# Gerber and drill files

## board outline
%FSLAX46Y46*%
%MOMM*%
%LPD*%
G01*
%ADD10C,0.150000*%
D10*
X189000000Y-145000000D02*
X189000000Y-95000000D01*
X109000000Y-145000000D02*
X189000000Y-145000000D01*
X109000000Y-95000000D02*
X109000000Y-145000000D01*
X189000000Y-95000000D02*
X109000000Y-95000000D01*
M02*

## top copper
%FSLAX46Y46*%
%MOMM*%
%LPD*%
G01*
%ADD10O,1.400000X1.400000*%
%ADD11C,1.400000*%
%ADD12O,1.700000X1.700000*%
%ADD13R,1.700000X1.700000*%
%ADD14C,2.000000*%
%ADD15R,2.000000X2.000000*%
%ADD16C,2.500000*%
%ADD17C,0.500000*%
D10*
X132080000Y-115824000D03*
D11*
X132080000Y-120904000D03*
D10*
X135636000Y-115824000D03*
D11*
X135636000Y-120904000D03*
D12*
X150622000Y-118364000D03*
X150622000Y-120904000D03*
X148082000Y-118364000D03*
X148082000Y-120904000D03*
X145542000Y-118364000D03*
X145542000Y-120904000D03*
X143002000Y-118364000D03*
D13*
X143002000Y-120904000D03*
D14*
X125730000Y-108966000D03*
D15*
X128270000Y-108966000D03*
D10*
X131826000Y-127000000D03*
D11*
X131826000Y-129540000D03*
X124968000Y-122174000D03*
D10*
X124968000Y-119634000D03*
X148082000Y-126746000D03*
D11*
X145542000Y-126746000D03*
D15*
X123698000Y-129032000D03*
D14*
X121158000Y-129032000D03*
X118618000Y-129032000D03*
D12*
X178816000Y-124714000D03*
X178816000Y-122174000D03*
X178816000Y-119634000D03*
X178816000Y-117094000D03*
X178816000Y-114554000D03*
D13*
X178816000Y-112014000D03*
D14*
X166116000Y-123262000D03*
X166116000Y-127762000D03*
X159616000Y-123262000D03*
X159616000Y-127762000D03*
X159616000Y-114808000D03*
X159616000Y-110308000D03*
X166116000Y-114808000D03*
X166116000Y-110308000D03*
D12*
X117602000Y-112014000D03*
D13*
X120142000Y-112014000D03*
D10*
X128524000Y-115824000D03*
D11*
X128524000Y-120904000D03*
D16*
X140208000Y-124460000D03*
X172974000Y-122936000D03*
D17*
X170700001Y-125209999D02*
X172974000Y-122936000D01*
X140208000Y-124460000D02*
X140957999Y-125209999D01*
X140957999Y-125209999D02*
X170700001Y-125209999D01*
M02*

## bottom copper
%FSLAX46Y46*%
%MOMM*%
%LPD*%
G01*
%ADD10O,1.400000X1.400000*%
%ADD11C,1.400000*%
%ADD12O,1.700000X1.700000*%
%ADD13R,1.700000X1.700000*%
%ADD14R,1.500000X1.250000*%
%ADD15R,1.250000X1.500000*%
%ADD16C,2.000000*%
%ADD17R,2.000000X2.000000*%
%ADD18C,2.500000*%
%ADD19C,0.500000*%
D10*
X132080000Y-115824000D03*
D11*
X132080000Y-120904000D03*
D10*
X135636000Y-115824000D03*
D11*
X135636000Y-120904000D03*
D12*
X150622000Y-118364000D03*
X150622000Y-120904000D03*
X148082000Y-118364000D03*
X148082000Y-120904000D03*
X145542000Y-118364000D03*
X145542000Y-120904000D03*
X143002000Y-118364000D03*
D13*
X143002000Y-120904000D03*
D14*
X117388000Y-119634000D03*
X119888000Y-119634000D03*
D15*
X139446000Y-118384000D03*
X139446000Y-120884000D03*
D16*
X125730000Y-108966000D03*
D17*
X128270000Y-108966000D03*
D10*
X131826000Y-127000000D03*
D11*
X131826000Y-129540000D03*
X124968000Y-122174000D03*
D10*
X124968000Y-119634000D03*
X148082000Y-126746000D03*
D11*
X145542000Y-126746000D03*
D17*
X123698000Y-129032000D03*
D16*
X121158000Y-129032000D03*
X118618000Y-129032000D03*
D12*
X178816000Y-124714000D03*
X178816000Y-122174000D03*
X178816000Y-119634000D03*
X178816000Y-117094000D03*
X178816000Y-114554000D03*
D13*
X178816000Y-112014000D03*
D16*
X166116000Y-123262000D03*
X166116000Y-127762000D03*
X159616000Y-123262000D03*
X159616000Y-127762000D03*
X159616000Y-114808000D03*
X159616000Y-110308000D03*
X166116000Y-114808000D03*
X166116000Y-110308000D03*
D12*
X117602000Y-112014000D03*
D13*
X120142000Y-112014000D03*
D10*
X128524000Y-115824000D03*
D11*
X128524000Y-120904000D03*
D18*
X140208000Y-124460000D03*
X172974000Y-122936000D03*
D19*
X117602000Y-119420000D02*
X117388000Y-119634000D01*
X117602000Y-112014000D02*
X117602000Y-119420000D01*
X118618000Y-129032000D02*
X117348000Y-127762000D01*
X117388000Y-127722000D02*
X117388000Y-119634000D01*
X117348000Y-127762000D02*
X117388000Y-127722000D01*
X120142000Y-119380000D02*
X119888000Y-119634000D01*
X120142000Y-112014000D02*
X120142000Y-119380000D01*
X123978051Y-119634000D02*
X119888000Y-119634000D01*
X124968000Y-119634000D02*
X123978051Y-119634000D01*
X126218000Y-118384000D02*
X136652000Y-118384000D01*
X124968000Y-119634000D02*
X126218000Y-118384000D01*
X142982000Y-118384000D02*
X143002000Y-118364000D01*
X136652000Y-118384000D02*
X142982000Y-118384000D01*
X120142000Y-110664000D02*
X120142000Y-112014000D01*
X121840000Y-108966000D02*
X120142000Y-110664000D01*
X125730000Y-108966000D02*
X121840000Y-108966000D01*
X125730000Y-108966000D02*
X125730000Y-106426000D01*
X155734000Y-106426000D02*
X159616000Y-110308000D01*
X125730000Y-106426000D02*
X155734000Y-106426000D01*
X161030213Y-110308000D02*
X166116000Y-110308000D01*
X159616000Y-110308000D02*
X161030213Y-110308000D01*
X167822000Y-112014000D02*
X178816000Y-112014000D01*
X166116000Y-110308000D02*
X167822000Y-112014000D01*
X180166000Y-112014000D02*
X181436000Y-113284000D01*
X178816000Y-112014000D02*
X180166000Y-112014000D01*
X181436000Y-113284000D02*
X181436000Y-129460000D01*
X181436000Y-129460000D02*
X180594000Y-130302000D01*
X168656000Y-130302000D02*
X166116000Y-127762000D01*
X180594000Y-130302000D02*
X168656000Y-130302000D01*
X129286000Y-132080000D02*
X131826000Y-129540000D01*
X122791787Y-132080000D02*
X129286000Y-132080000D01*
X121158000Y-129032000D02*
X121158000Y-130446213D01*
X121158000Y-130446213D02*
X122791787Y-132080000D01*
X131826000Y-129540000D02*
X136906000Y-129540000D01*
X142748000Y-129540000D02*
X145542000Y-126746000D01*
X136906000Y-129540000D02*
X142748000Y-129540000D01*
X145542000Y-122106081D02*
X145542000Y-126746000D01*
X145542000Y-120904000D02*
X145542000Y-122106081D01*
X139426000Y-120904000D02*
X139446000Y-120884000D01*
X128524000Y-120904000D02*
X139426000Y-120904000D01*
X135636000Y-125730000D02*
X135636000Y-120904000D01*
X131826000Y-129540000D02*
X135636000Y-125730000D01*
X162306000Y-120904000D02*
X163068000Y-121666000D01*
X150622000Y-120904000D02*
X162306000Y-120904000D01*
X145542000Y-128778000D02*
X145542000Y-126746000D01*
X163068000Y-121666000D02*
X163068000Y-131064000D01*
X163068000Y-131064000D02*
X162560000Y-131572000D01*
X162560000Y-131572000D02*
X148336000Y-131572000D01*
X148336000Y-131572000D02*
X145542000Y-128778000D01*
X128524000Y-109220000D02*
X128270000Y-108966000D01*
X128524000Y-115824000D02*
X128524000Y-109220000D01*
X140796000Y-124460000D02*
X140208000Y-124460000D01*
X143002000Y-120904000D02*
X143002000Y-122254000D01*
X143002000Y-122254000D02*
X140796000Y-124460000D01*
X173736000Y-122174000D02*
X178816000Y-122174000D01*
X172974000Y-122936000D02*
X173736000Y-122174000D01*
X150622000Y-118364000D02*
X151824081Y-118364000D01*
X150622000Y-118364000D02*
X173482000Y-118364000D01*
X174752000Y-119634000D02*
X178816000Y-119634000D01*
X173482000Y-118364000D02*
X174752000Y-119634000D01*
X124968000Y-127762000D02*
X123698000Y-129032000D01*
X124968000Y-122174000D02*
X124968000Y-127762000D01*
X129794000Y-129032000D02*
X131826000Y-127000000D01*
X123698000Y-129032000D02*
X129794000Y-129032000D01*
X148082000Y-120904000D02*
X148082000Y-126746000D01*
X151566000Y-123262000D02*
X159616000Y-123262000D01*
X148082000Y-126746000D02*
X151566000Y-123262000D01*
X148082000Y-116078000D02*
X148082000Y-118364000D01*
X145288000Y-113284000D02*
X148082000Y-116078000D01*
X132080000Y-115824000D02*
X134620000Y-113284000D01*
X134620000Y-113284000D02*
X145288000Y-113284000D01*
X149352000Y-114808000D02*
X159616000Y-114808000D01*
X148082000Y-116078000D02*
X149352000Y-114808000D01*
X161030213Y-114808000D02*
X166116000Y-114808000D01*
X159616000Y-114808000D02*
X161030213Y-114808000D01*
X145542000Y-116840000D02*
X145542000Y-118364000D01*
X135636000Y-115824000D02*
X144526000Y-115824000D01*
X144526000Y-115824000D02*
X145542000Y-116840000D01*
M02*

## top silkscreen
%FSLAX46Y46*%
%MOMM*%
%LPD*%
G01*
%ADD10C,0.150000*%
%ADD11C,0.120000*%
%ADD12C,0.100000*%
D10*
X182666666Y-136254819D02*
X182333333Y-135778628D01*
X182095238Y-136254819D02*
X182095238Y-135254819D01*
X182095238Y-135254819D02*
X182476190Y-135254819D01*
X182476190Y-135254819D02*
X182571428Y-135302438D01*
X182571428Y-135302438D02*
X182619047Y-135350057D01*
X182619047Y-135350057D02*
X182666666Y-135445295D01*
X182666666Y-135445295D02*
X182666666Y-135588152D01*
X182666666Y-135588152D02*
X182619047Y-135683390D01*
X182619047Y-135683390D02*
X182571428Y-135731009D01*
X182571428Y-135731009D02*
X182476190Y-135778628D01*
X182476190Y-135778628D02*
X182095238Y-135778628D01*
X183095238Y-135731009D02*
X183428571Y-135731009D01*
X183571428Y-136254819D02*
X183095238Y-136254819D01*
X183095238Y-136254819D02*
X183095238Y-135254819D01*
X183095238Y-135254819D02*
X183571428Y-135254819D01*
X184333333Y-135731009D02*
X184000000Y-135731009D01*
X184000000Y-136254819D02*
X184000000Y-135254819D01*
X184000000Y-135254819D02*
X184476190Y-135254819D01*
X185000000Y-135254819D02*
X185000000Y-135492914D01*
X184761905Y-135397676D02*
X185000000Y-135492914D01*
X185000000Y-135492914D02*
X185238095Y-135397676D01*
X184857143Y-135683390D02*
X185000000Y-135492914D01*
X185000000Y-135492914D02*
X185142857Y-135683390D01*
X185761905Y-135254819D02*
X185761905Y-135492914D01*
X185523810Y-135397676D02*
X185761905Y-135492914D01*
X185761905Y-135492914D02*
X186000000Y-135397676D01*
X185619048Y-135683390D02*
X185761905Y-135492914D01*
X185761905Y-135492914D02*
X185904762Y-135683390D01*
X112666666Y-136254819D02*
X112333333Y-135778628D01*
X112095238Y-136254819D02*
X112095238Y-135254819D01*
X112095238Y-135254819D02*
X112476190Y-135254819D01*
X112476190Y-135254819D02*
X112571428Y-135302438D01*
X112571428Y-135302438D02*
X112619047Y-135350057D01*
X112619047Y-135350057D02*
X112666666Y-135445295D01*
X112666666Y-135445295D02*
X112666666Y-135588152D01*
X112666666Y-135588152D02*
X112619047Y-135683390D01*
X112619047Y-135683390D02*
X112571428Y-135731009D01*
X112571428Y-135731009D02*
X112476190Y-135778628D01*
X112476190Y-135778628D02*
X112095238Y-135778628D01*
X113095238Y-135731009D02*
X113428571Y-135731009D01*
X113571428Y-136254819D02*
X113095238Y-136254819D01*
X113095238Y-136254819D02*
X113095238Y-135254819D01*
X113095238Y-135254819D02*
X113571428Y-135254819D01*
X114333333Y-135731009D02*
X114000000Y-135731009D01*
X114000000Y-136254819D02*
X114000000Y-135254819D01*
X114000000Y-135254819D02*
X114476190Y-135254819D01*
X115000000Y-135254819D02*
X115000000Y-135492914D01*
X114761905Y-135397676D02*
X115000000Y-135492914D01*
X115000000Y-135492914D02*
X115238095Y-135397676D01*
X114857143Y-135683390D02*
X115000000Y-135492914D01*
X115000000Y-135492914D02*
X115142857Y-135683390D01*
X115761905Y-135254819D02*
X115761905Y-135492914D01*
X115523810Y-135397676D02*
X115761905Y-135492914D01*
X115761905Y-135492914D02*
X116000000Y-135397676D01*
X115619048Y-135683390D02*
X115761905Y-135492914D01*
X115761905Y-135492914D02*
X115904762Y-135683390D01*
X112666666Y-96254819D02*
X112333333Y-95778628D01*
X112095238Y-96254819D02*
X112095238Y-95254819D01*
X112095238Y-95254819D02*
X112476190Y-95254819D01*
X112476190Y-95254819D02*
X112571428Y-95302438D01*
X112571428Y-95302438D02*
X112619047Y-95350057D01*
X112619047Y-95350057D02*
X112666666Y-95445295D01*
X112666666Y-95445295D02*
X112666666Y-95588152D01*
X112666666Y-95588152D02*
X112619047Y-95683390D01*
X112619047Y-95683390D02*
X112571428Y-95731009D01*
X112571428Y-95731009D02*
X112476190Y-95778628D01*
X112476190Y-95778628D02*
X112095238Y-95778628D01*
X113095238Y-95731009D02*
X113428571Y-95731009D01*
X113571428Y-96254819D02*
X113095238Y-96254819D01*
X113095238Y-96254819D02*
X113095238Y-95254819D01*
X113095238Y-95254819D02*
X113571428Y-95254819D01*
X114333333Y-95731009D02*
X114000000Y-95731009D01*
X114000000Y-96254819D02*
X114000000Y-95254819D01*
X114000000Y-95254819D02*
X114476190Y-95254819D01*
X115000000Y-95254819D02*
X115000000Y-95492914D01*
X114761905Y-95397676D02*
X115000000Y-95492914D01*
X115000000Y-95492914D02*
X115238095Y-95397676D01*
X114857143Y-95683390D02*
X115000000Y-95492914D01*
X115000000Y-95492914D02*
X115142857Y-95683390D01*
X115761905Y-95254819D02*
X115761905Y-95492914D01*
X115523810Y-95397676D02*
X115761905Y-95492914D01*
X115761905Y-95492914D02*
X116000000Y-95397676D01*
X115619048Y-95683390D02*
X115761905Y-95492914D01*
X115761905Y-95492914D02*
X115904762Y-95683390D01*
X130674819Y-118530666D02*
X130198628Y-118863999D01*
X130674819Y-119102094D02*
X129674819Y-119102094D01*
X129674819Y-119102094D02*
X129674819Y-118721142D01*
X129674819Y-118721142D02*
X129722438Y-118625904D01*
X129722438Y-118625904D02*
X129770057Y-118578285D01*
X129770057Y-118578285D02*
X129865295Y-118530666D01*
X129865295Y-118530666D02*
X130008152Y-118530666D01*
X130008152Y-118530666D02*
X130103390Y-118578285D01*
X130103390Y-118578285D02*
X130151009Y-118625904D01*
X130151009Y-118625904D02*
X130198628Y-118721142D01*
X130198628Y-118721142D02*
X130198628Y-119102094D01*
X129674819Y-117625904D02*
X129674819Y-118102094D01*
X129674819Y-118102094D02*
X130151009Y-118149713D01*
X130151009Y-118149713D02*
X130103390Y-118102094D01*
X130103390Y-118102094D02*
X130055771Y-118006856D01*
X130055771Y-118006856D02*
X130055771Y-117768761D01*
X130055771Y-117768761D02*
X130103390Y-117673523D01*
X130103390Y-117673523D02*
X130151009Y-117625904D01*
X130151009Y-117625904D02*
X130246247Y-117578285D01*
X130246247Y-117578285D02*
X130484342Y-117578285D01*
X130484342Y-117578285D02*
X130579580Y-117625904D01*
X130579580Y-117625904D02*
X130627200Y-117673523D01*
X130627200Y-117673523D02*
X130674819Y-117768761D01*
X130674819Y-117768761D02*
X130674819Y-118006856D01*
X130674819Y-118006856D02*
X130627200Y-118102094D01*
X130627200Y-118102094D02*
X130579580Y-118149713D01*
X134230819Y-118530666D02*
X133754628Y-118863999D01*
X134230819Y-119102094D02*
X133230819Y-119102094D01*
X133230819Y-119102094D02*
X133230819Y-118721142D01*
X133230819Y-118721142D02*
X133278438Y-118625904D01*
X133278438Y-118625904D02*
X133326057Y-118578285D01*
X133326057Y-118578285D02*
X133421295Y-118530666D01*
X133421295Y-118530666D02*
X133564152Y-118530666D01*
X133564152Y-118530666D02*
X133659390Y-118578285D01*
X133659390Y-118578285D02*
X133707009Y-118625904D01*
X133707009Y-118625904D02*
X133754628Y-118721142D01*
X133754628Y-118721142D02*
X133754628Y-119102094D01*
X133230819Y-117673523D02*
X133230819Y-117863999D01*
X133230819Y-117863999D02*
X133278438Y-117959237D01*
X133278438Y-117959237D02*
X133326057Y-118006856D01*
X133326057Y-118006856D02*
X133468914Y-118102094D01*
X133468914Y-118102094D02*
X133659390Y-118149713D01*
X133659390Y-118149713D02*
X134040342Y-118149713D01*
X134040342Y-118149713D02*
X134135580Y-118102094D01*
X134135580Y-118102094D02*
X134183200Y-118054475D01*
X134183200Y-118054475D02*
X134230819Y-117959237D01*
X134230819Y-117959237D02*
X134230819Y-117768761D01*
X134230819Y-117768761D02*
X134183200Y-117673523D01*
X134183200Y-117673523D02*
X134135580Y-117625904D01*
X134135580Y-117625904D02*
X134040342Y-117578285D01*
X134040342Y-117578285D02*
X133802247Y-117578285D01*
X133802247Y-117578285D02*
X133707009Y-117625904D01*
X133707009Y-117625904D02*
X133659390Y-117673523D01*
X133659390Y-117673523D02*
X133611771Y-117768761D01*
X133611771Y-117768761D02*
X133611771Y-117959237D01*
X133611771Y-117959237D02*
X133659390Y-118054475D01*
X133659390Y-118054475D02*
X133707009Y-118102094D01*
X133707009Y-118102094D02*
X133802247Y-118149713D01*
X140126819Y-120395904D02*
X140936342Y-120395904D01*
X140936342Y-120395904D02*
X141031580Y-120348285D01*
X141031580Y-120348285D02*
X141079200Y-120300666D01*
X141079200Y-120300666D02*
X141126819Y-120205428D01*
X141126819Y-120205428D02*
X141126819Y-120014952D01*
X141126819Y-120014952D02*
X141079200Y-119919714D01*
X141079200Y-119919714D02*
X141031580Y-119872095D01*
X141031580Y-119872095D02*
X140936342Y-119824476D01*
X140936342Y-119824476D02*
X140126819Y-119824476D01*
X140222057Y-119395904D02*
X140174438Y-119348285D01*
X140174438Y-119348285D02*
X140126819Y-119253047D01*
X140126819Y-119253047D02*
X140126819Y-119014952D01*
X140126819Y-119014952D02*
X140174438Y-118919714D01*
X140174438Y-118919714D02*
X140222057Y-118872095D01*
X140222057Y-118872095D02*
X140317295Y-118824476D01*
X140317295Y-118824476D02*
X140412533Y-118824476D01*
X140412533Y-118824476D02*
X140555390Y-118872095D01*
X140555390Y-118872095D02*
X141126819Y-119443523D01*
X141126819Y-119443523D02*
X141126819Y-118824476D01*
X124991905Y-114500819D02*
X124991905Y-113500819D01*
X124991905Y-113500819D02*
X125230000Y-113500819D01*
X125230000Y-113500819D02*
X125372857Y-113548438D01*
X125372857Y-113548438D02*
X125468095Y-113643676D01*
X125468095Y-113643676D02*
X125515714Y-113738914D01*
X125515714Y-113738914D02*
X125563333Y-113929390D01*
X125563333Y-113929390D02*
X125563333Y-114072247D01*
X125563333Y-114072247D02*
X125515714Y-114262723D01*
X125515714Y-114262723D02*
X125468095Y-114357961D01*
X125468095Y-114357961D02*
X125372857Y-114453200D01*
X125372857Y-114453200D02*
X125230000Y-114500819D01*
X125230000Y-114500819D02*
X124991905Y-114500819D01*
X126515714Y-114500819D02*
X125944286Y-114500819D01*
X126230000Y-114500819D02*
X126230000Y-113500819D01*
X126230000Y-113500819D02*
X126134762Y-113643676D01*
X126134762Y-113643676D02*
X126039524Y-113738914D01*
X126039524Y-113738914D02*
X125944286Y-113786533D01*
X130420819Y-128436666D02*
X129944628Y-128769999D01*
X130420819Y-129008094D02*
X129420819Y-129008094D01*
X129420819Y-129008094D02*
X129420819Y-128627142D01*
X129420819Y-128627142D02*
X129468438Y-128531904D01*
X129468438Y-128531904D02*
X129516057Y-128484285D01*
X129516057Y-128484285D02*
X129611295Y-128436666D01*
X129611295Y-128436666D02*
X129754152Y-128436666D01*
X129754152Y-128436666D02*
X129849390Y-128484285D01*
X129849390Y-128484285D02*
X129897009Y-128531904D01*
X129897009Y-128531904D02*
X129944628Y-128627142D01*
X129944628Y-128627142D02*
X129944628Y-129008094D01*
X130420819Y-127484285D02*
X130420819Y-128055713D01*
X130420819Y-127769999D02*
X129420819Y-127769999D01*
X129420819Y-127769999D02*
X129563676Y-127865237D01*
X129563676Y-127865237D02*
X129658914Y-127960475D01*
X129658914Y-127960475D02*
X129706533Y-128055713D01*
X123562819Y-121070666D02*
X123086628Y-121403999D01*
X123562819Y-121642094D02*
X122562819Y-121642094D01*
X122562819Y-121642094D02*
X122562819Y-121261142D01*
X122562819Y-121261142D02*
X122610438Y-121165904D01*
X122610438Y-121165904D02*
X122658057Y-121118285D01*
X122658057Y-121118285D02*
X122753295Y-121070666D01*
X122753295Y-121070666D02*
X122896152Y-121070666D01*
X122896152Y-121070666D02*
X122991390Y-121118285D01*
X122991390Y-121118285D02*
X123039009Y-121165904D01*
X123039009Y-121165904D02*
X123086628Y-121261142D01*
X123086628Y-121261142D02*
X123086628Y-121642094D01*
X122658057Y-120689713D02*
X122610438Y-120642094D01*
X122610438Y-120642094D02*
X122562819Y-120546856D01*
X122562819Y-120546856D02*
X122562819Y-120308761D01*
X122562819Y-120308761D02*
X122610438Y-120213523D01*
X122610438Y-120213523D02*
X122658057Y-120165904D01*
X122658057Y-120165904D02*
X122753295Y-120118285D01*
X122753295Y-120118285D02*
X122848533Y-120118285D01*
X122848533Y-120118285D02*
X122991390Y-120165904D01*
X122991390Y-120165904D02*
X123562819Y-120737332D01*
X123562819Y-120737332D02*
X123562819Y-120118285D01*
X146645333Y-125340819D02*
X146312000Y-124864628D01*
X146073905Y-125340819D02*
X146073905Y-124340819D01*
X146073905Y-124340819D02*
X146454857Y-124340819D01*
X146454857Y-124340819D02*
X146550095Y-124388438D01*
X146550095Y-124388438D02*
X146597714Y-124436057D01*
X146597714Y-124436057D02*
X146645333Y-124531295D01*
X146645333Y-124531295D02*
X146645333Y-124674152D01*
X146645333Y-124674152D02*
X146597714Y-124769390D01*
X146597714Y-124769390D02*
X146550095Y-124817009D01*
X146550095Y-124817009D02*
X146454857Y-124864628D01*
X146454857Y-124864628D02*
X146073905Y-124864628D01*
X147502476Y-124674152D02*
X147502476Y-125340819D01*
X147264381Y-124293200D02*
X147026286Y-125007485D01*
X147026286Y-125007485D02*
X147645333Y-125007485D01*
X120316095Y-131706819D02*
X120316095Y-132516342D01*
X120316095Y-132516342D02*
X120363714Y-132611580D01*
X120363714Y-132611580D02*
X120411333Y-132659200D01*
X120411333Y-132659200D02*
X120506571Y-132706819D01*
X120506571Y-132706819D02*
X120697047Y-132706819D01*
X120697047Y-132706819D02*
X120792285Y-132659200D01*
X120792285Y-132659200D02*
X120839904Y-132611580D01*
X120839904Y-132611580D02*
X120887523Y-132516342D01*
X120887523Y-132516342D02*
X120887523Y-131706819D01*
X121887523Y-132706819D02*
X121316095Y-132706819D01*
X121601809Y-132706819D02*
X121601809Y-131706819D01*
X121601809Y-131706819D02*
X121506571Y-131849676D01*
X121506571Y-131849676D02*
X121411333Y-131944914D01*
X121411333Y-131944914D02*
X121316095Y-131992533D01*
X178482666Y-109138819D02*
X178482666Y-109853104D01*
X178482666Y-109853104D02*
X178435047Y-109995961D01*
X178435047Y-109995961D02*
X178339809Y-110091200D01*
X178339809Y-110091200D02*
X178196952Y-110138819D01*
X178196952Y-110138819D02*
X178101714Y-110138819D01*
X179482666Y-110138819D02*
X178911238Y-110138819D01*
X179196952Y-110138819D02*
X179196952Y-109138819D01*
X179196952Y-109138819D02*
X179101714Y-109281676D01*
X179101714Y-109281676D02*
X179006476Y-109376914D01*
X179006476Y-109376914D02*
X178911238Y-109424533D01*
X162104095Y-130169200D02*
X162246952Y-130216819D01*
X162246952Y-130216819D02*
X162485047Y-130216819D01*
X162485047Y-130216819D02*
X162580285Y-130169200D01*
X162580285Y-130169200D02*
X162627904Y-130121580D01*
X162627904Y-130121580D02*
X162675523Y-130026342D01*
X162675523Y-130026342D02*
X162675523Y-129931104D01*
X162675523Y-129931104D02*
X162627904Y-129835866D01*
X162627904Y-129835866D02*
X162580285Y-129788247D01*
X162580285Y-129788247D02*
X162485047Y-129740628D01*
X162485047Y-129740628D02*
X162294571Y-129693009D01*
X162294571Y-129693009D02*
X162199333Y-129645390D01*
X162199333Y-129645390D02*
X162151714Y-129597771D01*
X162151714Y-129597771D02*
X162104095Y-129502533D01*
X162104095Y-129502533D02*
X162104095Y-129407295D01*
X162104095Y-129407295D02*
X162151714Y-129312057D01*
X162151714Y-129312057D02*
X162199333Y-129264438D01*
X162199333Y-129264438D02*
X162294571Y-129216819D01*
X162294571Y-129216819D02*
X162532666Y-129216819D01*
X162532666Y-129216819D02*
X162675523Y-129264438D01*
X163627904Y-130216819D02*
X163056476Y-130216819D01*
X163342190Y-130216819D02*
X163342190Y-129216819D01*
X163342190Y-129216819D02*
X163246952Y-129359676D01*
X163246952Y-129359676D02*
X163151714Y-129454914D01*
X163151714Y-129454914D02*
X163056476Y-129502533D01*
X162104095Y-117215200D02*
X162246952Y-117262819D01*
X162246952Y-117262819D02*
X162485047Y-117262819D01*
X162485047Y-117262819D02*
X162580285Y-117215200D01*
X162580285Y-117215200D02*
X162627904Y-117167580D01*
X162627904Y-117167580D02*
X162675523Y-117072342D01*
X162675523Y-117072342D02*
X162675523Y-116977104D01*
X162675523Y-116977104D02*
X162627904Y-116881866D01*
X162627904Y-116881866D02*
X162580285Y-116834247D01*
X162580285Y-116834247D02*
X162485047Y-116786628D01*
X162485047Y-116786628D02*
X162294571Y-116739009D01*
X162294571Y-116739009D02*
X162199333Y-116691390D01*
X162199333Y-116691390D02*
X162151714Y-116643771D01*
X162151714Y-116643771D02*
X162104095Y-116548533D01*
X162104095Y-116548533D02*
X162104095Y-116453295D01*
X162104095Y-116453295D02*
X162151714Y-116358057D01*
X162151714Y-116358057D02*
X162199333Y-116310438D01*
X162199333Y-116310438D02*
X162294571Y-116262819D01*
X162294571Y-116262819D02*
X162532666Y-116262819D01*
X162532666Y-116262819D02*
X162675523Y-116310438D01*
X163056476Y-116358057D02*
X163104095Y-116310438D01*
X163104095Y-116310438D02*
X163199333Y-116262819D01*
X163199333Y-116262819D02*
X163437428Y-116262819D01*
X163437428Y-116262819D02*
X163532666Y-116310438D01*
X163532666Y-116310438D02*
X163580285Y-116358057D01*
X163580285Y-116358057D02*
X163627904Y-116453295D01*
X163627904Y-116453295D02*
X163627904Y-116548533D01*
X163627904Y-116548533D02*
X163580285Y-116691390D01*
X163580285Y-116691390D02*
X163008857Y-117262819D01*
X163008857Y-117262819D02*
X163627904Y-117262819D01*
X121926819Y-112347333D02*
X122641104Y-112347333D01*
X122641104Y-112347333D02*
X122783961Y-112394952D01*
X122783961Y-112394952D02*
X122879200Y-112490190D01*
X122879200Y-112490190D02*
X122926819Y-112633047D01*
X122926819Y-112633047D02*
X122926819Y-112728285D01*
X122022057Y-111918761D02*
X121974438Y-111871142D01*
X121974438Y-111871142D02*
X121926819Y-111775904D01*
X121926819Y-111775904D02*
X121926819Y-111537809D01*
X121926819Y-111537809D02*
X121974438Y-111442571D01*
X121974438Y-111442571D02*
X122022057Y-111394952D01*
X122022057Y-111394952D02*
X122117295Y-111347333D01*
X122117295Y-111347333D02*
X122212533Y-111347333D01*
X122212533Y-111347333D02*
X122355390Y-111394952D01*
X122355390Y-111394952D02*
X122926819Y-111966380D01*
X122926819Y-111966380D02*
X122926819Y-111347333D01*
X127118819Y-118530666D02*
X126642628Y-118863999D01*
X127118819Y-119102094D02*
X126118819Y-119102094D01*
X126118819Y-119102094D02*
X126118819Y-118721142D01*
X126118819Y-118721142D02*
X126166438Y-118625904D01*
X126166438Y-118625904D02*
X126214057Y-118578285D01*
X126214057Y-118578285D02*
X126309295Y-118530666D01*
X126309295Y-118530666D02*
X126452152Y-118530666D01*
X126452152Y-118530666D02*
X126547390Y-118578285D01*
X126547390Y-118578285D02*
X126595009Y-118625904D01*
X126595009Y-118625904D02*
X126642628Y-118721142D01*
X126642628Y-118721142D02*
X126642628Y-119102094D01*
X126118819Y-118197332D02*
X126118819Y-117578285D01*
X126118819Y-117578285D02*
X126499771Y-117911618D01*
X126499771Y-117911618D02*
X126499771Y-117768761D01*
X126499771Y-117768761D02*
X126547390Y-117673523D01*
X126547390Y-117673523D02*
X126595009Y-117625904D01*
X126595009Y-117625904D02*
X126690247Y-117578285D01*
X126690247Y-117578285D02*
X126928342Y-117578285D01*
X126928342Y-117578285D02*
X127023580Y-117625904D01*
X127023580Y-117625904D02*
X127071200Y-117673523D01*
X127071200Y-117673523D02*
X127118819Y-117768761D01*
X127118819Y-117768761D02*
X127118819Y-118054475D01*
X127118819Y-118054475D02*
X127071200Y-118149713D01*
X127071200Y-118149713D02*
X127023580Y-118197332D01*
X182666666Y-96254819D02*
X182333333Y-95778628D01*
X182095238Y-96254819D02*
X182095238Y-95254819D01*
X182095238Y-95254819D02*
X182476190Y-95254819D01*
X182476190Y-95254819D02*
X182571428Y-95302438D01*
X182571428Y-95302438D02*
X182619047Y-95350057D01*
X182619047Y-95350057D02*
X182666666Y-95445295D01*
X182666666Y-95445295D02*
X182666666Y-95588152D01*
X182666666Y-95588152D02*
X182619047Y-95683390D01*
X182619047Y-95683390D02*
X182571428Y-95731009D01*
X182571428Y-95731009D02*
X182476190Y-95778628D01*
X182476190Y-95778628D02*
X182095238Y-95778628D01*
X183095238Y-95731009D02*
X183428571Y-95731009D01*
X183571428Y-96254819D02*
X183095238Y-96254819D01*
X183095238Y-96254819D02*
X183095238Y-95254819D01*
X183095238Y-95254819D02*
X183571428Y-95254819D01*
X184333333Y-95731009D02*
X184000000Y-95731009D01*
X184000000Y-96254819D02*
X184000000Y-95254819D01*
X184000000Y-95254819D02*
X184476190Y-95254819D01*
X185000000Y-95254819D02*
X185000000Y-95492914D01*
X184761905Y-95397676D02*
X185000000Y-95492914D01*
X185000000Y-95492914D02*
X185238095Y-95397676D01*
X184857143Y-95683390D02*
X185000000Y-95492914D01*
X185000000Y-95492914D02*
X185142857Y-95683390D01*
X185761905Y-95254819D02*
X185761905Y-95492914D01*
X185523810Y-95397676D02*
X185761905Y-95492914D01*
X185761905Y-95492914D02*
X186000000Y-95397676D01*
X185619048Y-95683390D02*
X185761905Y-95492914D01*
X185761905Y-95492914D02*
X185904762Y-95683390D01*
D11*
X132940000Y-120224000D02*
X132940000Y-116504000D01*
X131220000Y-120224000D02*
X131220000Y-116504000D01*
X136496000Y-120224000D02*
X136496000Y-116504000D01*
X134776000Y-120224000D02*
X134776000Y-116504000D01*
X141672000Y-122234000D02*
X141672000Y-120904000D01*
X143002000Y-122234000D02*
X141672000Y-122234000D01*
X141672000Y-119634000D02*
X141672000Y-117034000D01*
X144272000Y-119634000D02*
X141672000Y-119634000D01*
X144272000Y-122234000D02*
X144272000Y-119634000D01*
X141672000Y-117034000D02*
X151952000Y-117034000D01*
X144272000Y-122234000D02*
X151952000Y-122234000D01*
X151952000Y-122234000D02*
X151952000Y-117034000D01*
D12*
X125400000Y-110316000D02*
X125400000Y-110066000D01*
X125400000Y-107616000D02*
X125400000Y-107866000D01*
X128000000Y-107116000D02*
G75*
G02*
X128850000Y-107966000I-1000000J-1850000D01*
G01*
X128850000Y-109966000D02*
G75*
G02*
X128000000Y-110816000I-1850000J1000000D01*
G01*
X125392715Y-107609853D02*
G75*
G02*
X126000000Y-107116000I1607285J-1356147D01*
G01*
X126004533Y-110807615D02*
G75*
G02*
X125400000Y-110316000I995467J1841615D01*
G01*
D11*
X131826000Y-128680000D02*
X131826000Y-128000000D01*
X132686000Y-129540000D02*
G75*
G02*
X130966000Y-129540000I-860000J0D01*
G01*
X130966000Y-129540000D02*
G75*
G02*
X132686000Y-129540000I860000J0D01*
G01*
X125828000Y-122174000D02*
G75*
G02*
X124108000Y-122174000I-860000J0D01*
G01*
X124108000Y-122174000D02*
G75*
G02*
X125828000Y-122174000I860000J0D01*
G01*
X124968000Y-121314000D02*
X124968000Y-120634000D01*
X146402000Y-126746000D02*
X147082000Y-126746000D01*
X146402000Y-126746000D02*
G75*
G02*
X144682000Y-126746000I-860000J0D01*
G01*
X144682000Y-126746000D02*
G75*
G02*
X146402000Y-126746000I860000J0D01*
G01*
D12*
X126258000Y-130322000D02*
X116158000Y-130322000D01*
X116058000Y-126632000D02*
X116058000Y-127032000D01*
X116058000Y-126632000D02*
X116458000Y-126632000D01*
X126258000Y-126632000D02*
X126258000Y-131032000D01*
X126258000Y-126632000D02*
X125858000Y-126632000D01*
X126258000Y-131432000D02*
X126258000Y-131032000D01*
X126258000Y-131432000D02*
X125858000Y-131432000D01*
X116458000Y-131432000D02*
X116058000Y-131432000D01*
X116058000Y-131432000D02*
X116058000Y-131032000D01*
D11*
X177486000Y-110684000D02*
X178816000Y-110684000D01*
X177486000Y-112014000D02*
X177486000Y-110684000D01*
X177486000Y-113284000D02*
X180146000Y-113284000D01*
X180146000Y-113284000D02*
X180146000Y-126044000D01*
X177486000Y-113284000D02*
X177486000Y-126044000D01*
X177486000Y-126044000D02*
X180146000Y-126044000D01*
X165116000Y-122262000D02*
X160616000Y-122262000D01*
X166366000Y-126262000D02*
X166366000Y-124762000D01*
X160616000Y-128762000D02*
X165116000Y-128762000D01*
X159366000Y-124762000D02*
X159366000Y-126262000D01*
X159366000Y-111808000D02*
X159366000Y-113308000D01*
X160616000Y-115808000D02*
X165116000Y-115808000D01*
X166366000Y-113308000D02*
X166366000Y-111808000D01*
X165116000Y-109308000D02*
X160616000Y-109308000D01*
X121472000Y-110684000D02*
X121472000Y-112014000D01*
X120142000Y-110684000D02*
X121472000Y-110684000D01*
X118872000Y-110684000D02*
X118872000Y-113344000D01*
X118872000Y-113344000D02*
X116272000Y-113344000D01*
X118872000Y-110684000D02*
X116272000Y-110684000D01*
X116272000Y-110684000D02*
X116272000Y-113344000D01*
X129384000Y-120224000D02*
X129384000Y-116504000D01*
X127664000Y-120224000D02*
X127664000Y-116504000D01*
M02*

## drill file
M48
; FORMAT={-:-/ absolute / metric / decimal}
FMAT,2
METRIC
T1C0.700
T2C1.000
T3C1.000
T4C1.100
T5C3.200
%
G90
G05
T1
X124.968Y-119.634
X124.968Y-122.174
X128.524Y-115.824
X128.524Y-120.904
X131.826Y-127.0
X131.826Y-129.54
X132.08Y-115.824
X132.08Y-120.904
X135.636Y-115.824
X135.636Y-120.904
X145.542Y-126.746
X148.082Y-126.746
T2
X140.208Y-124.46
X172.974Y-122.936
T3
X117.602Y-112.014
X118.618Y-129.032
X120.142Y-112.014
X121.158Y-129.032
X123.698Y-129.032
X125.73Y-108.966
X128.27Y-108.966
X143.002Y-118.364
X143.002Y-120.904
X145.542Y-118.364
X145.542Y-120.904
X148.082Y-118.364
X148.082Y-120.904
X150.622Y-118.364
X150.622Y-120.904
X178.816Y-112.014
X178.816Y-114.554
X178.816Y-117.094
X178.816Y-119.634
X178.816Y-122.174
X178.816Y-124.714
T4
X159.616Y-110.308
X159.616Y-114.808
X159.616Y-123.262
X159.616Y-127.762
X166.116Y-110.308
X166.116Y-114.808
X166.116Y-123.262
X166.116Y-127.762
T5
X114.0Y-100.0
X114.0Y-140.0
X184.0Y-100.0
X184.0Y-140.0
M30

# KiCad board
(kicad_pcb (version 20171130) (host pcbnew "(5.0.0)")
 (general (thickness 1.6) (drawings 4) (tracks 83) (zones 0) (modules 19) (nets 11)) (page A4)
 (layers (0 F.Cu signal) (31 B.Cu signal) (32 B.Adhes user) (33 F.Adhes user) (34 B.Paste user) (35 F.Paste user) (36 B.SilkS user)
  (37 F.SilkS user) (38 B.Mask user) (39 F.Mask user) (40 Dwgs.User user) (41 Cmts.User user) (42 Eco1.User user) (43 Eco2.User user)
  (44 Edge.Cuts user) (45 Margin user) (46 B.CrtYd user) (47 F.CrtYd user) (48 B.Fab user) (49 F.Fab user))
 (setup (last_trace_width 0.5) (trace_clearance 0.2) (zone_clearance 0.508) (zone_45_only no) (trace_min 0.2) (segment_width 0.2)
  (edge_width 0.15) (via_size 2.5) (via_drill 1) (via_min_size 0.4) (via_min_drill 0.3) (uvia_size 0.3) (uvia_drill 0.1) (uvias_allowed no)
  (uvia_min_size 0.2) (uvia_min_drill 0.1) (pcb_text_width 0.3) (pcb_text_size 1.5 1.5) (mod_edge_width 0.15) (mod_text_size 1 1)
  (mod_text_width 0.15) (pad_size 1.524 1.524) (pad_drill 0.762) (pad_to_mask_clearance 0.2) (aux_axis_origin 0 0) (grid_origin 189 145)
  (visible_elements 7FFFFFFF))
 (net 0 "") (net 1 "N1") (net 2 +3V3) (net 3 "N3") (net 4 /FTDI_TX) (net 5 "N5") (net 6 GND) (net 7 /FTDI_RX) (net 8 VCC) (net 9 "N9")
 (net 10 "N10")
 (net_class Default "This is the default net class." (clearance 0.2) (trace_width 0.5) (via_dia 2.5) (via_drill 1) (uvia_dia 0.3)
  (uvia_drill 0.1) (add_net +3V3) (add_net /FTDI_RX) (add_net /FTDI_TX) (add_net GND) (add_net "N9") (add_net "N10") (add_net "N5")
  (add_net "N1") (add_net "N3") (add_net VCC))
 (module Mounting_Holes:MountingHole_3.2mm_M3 (layer F.Cu) (at 184 140)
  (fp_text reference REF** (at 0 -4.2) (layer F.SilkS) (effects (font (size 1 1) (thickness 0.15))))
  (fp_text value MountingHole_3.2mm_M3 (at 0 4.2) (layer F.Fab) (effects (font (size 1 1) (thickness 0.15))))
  (pad 1 np_thru_hole circle (at 0 0) (size 3.2 3.2) (drill 3.2) (layers *.Cu *.Mask)))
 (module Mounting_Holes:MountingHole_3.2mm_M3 (layer F.Cu) (at 114 140)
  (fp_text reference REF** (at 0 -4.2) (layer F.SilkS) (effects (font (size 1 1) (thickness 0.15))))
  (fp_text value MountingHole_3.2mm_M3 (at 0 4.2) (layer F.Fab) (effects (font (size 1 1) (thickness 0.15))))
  (pad 1 np_thru_hole circle (at 0 0) (size 3.2 3.2) (drill 3.2) (layers *.Cu *.Mask)))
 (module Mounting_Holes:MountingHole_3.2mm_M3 (layer F.Cu) (at 114 100)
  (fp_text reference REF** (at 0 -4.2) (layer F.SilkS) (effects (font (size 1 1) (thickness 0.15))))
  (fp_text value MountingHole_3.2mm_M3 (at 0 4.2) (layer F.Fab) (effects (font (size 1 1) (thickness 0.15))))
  (pad 1 np_thru_hole circle (at 0 0) (size 3.2 3.2) (drill 3.2) (layers *.Cu *.Mask)))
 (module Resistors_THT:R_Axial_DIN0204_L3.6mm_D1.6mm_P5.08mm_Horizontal (layer F.Cu) (at 132.08 120.904 90)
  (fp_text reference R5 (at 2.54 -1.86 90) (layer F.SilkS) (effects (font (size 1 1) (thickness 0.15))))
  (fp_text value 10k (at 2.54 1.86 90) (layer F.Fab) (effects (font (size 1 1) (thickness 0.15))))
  (fp_line (start 0.68 0.86) (end 4.4 0.86) (layer F.SilkS) (width 0.12))
  (fp_line (start 0.68 -0.86) (end 4.4 -0.86) (layer F.SilkS) (width 0.12))
  (pad 2 thru_hole oval (at 5.08 0 90) (size 1.4 1.4) (drill 0.7) (layers *.Cu *.Mask) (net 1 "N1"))
  (pad 1 thru_hole circle (at 0 0 90) (size 1.4 1.4) (drill 0.7) (layers *.Cu *.Mask) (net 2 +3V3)))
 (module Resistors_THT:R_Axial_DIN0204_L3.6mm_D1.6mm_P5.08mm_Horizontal (layer F.Cu) (at 135.636 120.904 90)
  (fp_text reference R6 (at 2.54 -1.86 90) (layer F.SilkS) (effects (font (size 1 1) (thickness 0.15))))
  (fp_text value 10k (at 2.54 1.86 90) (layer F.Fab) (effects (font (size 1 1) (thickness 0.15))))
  (fp_line (start 0.68 0.86) (end 4.4 0.86) (layer F.SilkS) (width 0.12))
  (fp_line (start 0.68 -0.86) (end 4.4 -0.86) (layer F.SilkS) (width 0.12))
  (pad 2 thru_hole oval (at 5.08 0 90) (size 1.4 1.4) (drill 0.7) (layers *.Cu *.Mask) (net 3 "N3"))
  (pad 1 thru_hole circle (at 0 0 90) (size 1.4 1.4) (drill 0.7) (layers *.Cu *.Mask) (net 2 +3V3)))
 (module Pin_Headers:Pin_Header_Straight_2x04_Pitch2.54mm (layer F.Cu) (at 143.002 120.904 90)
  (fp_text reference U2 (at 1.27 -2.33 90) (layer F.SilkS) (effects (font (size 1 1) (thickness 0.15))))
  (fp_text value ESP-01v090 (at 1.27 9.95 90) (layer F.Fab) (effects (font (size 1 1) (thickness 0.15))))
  (fp_line (start -1.33 -1.33) (end 0 -1.33) (layer F.SilkS) (width 0.12))
  (fp_line (start -1.33 0) (end -1.33 -1.33) (layer F.SilkS) (width 0.12))
  (fp_line (start 1.27 -1.33) (end 3.87 -1.33) (layer F.SilkS) (width 0.12))
  (fp_line (start 1.27 1.27) (end 1.27 -1.33) (layer F.SilkS) (width 0.12))
  (fp_line (start -1.33 1.27) (end 1.27 1.27) (layer F.SilkS) (width 0.12))
  (fp_line (start 3.87 -1.33) (end 3.87 8.95) (layer F.SilkS) (width 0.12))
  (fp_line (start -1.33 1.27) (end -1.33 8.95) (layer F.SilkS) (width 0.12))
  (fp_line (start -1.33 8.95) (end 3.87 8.95) (layer F.SilkS) (width 0.12))
  (pad 8 thru_hole oval (at 2.54 7.62 90) (size 1.7 1.7) (drill 1) (layers *.Cu *.Mask) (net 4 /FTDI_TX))
  (pad 7 thru_hole oval (at 0 7.62 90) (size 1.7 1.7) (drill 1) (layers *.Cu *.Mask) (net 2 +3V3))
  (pad 6 thru_hole oval (at 2.54 5.08 90) (size 1.7 1.7) (drill 1) (layers *.Cu *.Mask) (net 1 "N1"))
  (pad 5 thru_hole oval (at 0 5.08 90) (size 1.7 1.7) (drill 1) (layers *.Cu *.Mask) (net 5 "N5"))
  (pad 4 thru_hole oval (at 2.54 2.54 90) (size 1.7 1.7) (drill 1) (layers *.Cu *.Mask) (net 3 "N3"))
  (pad 3 thru_hole oval (at 0 2.54 90) (size 1.7 1.7) (drill 1) (layers *.Cu *.Mask) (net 2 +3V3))
  (pad 2 thru_hole oval (at 2.54 0 90) (size 1.7 1.7) (drill 1) (layers *.Cu *.Mask) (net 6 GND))
  (pad 1 thru_hole rect (at 0 0 90) (size 1.7 1.7) (drill 1) (layers *.Cu *.Mask) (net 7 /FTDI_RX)))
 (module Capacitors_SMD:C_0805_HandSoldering (layer B.Cu) (at 118.638 119.634)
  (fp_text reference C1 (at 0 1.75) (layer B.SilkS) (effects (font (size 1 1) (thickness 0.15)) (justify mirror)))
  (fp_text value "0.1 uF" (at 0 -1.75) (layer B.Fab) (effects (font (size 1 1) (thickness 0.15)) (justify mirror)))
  (pad 1 smd rect (at -1.25 0) (size 1.5 1.25) (layers B.Cu B.Paste B.Mask) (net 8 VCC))
  (pad 2 smd rect (at 1.25 0) (size 1.5 1.25) (layers B.Cu B.Paste B.Mask) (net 6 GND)))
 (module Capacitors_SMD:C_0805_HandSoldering (layer B.Cu) (at 139.446 119.634 90)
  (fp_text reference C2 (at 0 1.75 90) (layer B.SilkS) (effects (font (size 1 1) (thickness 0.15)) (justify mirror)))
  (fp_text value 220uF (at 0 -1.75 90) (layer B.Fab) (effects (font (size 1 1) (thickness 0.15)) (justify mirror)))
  (pad 2 smd rect (at 1.25 0 90) (size 1.5 1.25) (layers B.Cu B.Paste B.Mask) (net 6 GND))
  (pad 1 smd rect (at -1.25 0 90) (size 1.5 1.25) (layers B.Cu B.Paste B.Mask) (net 2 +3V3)))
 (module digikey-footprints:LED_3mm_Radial (layer F.Cu) (at 125.73 108.966 180)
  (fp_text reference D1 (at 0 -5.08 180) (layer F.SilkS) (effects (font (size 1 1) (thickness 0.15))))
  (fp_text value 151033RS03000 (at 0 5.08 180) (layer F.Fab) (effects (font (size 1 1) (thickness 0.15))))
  (fp_line (start 0.33 -1.35) (end 0.33 -1.1) (layer F.SilkS) (width 0.1))
  (fp_line (start 0.33 1.35) (end 0.33 1.1) (layer F.SilkS) (width 0.1))
  (fp_arc (start -1.27 0) (end -3.12 1) (angle -33.21396116) (layer F.SilkS) (width 0.1))
  (fp_arc (start -1.27 0) (end -2.27 -1.85) (angle -33.21396116) (layer F.SilkS) (width 0.1))
  (fp_arc (start -1.27 0) (end -0.27 1.85) (angle -21.45098095) (layer F.SilkS) (width 0.1))
  (fp_arc (start -1.27 0) (end 0.33 -1.35) (angle -21.45098095) (layer F.SilkS) (width 0.1))
  (pad 2 thru_hole circle (at 0 0 180) (size 2 2) (drill 1) (layers *.Cu *.Mask) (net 6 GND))
  (pad 1 thru_hole rect (at -2.54 0 180) (size 2 2) (drill 1) (layers *.Cu *.Mask) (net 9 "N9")))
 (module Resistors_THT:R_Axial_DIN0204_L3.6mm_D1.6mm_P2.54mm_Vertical (layer F.Cu) (at 131.826 129.54 90)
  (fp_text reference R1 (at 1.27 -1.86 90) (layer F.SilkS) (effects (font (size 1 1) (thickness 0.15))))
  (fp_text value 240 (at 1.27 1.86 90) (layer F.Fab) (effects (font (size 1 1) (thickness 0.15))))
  (fp_line (start 0.86 0) (end 1.54 0) (layer F.SilkS) (width 0.12))
  (fp_circle (center 0 0) (end 0.86 0) (layer F.SilkS) (width 0.12))
  (pad 2 thru_hole oval (at 2.54 0 90) (size 1.4 1.4) (drill 0.7) (layers *.Cu *.Mask) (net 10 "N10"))
  (pad 1 thru_hole circle (at 0 0 90) (size 1.4 1.4) (drill 0.7) (layers *.Cu *.Mask) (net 2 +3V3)))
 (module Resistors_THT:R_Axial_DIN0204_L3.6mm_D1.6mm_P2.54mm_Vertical (layer F.Cu) (at 124.968 122.174 90)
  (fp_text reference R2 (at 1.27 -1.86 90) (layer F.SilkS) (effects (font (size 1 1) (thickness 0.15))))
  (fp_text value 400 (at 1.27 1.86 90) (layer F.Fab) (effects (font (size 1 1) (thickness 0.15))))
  (fp_circle (center 0 0) (end 0.86 0) (layer F.SilkS) (width 0.12))
  (fp_line (start 0.86 0) (end 1.54 0) (layer F.SilkS) (width 0.12))
  (pad 1 thru_hole circle (at 0 0 90) (size 1.4 1.4) (drill 0.7) (layers *.Cu *.Mask) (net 10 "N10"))
  (pad 2 thru_hole oval (at 2.54 0 90) (size 1.4 1.4) (drill 0.7) (layers *.Cu *.Mask) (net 6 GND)))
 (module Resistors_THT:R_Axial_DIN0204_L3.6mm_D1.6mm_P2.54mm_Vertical (layer F.Cu) (at 145.542 126.746)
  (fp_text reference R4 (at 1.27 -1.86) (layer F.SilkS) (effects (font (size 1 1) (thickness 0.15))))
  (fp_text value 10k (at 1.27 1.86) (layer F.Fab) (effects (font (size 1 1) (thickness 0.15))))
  (fp_line (start 0.86 0) (end 1.54 0) (layer F.SilkS) (width 0.12))
  (fp_circle (center 0 0) (end 0.86 0) (layer F.SilkS) (width 0.12))
  (pad 2 thru_hole oval (at 2.54 0) (size 1.4 1.4) (drill 0.7) (layers *.Cu *.Mask) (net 5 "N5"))
  (pad 1 thru_hole circle (at 0 0) (size 1.4 1.4) (drill 0.7) (layers *.Cu *.Mask) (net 2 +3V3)))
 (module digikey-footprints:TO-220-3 (layer F.Cu) (at 123.698 129.032 180)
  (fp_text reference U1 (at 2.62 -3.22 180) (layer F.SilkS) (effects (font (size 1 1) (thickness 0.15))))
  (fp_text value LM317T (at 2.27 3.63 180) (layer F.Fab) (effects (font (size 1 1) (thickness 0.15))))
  (fp_line (start -2.56 -1.29) (end 7.54 -1.29) (layer F.SilkS) (width 0.1))
  (fp_line (start 7.64 2.4) (end 7.64 2) (layer F.SilkS) (width 0.1))
  (fp_line (start 7.64 2.4) (end 7.24 2.4) (layer F.SilkS) (width 0.1))
  (fp_line (start -2.56 2.4) (end -2.56 -2) (layer F.SilkS) (width 0.1))
  (fp_line (start -2.56 2.4) (end -2.16 2.4) (layer F.SilkS) (width 0.1))
  (fp_line (start -2.56 -2.4) (end -2.56 -2) (layer F.SilkS) (width 0.1))
  (fp_line (start -2.56 -2.4) (end -2.16 -2.4) (layer F.SilkS) (width 0.1))
  (fp_line (start 7.24 -2.4) (end 7.64 -2.4) (layer F.SilkS) (width 0.1))
  (fp_line (start 7.64 -2.4) (end 7.64 -2) (layer F.SilkS) (width 0.1))
  (pad 1 thru_hole rect (at 0 0 180) (size 2 2) (drill 1) (layers *.Cu *.Mask) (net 10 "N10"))
  (pad 2 thru_hole circle (at 2.54 0 180) (size 2 2) (drill 1) (layers *.Cu *.Mask) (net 2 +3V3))
  (pad 3 thru_hole circle (at 5.08 0 180) (size 2 2) (drill 1) (layers *.Cu *.Mask) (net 8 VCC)))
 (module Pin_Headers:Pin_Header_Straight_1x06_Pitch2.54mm (layer F.Cu) (at 178.816 112.014)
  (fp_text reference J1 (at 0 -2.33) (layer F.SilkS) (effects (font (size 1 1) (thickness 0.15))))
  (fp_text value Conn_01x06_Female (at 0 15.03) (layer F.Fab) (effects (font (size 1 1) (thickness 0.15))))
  (fp_line (start -1.33 -1.33) (end 0 -1.33) (layer F.SilkS) (width 0.12))
  (fp_line (start -1.33 0) (end -1.33 -1.33) (layer F.SilkS) (width 0.12))
  (fp_line (start -1.33 1.27) (end 1.33 1.27) (layer F.SilkS) (width 0.12))
  (fp_line (start 1.33 1.27) (end 1.33 14.03) (layer F.SilkS) (width 0.12))
  (fp_line (start -1.33 1.27) (end -1.33 14.03) (layer F.SilkS) (width 0.12))
  (fp_line (start -1.33 14.03) (end 1.33 14.03) (layer F.SilkS) (width 0.12))
  (pad 6 thru_hole oval (at 0 12.7) (size 1.7 1.7) (drill 1) (layers *.Cu *.Mask))
  (pad 5 thru_hole oval (at 0 10.16) (size 1.7 1.7) (drill 1) (layers *.Cu *.Mask) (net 7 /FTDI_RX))
  (pad 4 thru_hole oval (at 0 7.62) (size 1.7 1.7) (drill 1) (layers *.Cu *.Mask) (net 4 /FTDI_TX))
  (pad 3 thru_hole oval (at 0 5.08) (size 1.7 1.7) (drill 1) (layers *.Cu *.Mask))
  (pad 2 thru_hole oval (at 0 2.54) (size 1.7 1.7) (drill 1) (layers *.Cu *.Mask))
  (pad 1 thru_hole rect (at 0 0) (size 1.7 1.7) (drill 1) (layers *.Cu *.Mask) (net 6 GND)))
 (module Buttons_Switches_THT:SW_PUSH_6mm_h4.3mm (layer F.Cu) (at 166.116 127.762 180)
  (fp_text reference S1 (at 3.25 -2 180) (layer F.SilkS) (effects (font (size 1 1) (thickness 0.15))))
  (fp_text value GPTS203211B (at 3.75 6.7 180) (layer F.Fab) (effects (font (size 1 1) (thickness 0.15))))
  (fp_line (start 1 5.5) (end 5.5 5.5) (layer F.SilkS) (width 0.12))
  (fp_line (start -0.25 1.5) (end -0.25 3) (layer F.SilkS) (width 0.12))
  (fp_line (start 5.5 -1) (end 1 -1) (layer F.SilkS) (width 0.12))
  (fp_line (start 6.75 3) (end 6.75 1.5) (layer F.SilkS) (width 0.12))
  (pad 2 thru_hole circle (at 0 4.5 270) (size 2 2) (drill 1.1) (layers *.Cu *.Mask) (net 5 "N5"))
  (pad 1 thru_hole circle (at 0 0 270) (size 2 2) (drill 1.1) (layers *.Cu *.Mask) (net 6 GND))
  (pad 2 thru_hole circle (at 6.5 4.5 270) (size 2 2) (drill 1.1) (layers *.Cu *.Mask) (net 5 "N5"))
  (pad 1 thru_hole circle (at 6.5 0 270) (size 2 2) (drill 1.1) (layers *.Cu *.Mask) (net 6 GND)))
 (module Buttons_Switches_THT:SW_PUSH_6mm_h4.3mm (layer F.Cu) (at 166.116 114.808 180)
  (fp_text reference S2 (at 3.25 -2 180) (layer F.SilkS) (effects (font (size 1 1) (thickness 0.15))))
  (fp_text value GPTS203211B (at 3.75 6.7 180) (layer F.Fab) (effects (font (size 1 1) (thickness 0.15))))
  (fp_line (start 6.75 3) (end 6.75 1.5) (layer F.SilkS) (width 0.12))
  (fp_line (start 5.5 -1) (end 1 -1) (layer F.SilkS) (width 0.12))
  (fp_line (start -0.25 1.5) (end -0.25 3) (layer F.SilkS) (width 0.12))
  (fp_line (start 1 5.5) (end 5.5 5.5) (layer F.SilkS) (width 0.12))
  (pad 1 thru_hole circle (at 6.5 0 270) (size 2 2) (drill 1.1) (layers *.Cu *.Mask) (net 1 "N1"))
  (pad 2 thru_hole circle (at 6.5 4.5 270) (size 2 2) (drill 1.1) (layers *.Cu *.Mask) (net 6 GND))
  (pad 1 thru_hole circle (at 0 0 270) (size 2 2) (drill 1.1) (layers *.Cu *.Mask) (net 1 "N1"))
  (pad 2 thru_hole circle (at 0 4.5 270) (size 2 2) (drill 1.1) (layers *.Cu *.Mask) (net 6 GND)))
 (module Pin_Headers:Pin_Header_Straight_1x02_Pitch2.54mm (layer F.Cu) (at 120.142 112.014 270)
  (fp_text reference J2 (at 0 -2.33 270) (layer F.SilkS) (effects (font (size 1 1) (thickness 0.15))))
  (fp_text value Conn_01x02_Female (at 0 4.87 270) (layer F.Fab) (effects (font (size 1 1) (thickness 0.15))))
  (fp_line (start -1.33 -1.33) (end 0 -1.33) (layer F.SilkS) (width 0.12))
  (fp_line (start -1.33 0) (end -1.33 -1.33) (layer F.SilkS) (width 0.12))
  (fp_line (start -1.33 1.27) (end 1.33 1.27) (layer F.SilkS) (width 0.12))
  (fp_line (start 1.33 1.27) (end 1.33 3.87) (layer F.SilkS) (width 0.12))
  (fp_line (start -1.33 1.27) (end -1.33 3.87) (layer F.SilkS) (width 0.12))
  (fp_line (start -1.33 3.87) (end 1.33 3.87) (layer F.SilkS) (width 0.12))
  (pad 2 thru_hole oval (at 0 2.54 270) (size 1.7 1.7) (drill 1) (layers *.Cu *.Mask) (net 8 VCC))
  (pad 1 thru_hole rect (at 0 0 270) (size 1.7 1.7) (drill 1) (layers *.Cu *.Mask) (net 6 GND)))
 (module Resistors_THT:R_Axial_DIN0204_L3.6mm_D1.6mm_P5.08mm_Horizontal (layer F.Cu) (at 128.524 120.904 90)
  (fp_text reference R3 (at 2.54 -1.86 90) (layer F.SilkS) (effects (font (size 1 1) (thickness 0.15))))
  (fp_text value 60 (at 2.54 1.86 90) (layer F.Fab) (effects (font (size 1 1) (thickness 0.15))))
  (fp_line (start 0.68 0.86) (end 4.4 0.86) (layer F.SilkS) (width 0.12))
  (fp_line (start 0.68 -0.86) (end 4.4 -0.86) (layer F.SilkS) (width 0.12))
  (pad 2 thru_hole oval (at 5.08 0 90) (size 1.4 1.4) (drill 0.7) (layers *.Cu *.Mask) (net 9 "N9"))
  (pad 1 thru_hole circle (at 0 0 90) (size 1.4 1.4) (drill 0.7) (layers *.Cu *.Mask) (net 2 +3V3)))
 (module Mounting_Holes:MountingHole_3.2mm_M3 (layer F.Cu) (at 184 100)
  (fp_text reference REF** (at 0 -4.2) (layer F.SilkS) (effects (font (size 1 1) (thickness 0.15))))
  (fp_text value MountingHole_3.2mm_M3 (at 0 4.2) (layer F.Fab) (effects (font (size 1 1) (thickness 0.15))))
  (pad 1 np_thru_hole circle (at 0 0) (size 3.2 3.2) (drill 3.2) (layers *.Cu *.Mask)))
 (gr_line (start 189 145) (end 189 95) (layer Edge.Cuts) (width 0.15))
 (gr_line (start 109 145) (end 189 145) (layer Edge.Cuts) (width 0.15))
 (gr_line (start 109 95) (end 109 145) (layer Edge.Cuts) (width 0.15))
 (gr_line (start 189 95) (end 109 95) (layer Edge.Cuts) (width 0.15))
 (segment (start 117.602 119.42) (end 117.388 119.634) (width 0.5) (layer B.Cu) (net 8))
 (segment (start 117.602 112.014) (end 117.602 119.42) (width 0.5) (layer B.Cu) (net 8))
 (segment (start 118.618 129.032) (end 117.348 127.762) (width 0.5) (layer B.Cu) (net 8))
 (segment (start 117.388 127.722) (end 117.388 119.634) (width 0.5) (layer B.Cu) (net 8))
 (segment (start 117.348 127.762) (end 117.388 127.722) (width 0.5) (layer B.Cu) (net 8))
 (segment (start 120.142 119.38) (end 119.888 119.634) (width 0.5) (layer B.Cu) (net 6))
 (segment (start 120.142 112.014) (end 120.142 119.38) (width 0.5) (layer B.Cu) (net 6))
 (segment (start 123.978051 119.634) (end 119.888 119.634) (width 0.5) (layer B.Cu) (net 6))
 (segment (start 124.968 119.634) (end 123.978051 119.634) (width 0.5) (layer B.Cu) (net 6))
 (segment (start 126.218 118.384) (end 136.652 118.384) (width 0.5) (layer B.Cu) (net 6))
 (segment (start 124.968 119.634) (end 126.218 118.384) (width 0.5) (layer B.Cu) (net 6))
 (segment (start 142.982 118.384) (end 143.002 118.364) (width 0.5) (layer B.Cu) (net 6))
 (segment (start 136.652 118.384) (end 142.982 118.384) (width 0.5) (layer B.Cu) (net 6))
 (segment (start 120.142 110.664) (end 120.142 112.014) (width 0.5) (layer B.Cu) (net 6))
 (segment (start 121.84 108.966) (end 120.142 110.664) (width 0.5) (layer B.Cu) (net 6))
 (segment (start 125.73 108.966) (end 121.84 108.966) (width 0.5) (layer B.Cu) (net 6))
 (segment (start 125.73 108.966) (end 125.73 106.426) (width 0.5) (layer B.Cu) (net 6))
 (segment (start 155.734 106.426) (end 159.616 110.308) (width 0.5) (layer B.Cu) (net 6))
 (segment (start 125.73 106.426) (end 155.734 106.426) (width 0.5) (layer B.Cu) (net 6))
 (segment (start 161.030213 110.308) (end 166.116 110.308) (width 0.5) (layer B.Cu) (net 6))
 (segment (start 159.616 110.308) (end 161.030213 110.308) (width 0.5) (layer B.Cu) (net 6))
 (segment (start 167.822 112.014) (end 178.816 112.014) (width 0.5) (layer B.Cu) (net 6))
 (segment (start 166.116 110.308) (end 167.822 112.014) (width 0.5) (layer B.Cu) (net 6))
 (segment (start 180.166 112.014) (end 181.436 113.284) (width 0.5) (layer B.Cu) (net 6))
 (segment (start 178.816 112.014) (end 180.166 112.014) (width 0.5) (layer B.Cu) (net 6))
 (segment (start 181.436 113.284) (end 181.436 129.46) (width 0.5) (layer B.Cu) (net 6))
 (segment (start 181.436 129.46) (end 180.594 130.302) (width 0.5) (layer B.Cu) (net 6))
 (segment (start 168.656 130.302) (end 166.116 127.762) (width 0.5) (layer B.Cu) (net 6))
 (segment (start 180.594 130.302) (end 168.656 130.302) (width 0.5) (layer B.Cu) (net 6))
 (segment (start 129.286 132.08) (end 131.826 129.54) (width 0.5) (layer B.Cu) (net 2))
 (segment (start 122.791787 132.08) (end 129.286 132.08) (width 0.5) (layer B.Cu) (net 2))
 (segment (start 121.158 129.032) (end 121.158 130.446213) (width 0.5) (layer B.Cu) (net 2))
 (segment (start 121.158 130.446213) (end 122.791787 132.08) (width 0.5) (layer B.Cu) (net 2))
 (segment (start 131.826 129.54) (end 136.906 129.54) (width 0.5) (layer B.Cu) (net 2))
 (segment (start 142.748 129.54) (end 145.542 126.746) (width 0.5) (layer B.Cu) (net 2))
 (segment (start 136.906 129.54) (end 142.748 129.54) (width 0.5) (layer B.Cu) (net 2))
 (segment (start 145.542 122.106081) (end 145.542 126.746) (width 0.5) (layer B.Cu) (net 2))
 (segment (start 145.542 120.904) (end 145.542 122.106081) (width 0.5) (layer B.Cu) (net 2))
 (segment (start 139.426 120.904) (end 139.446 120.884) (width 0.5) (layer B.Cu) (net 2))
 (segment (start 128.524 120.904) (end 139.426 120.904) (width 0.5) (layer B.Cu) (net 2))
 (segment (start 135.636 125.73) (end 135.636 120.904) (width 0.5) (layer B.Cu) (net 2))
 (segment (start 131.826 129.54) (end 135.636 125.73) (width 0.5) (layer B.Cu) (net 2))
 (segment (start 162.306 120.904) (end 163.068 121.666) (width 0.5) (layer B.Cu) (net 2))
 (segment (start 150.622 120.904) (end 162.306 120.904) (width 0.5) (layer B.Cu) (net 2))
 (segment (start 145.542 128.778) (end 145.542 126.746) (width 0.5) (layer B.Cu) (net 2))
 (segment (start 163.068 121.666) (end 163.068 131.064) (width 0.5) (layer B.Cu) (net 2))
 (segment (start 163.068 131.064) (end 162.56 131.572) (width 0.5) (layer B.Cu) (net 2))
 (segment (start 162.56 131.572) (end 148.336 131.572) (width 0.5) (layer B.Cu) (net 2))
 (segment (start 148.336 131.572) (end 145.542 128.778) (width 0.5) (layer B.Cu) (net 2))
 (segment (start 128.524 109.22) (end 128.27 108.966) (width 0.5) (layer B.Cu) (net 9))
 (segment (start 128.524 115.824) (end 128.524 109.22) (width 0.5) (layer B.Cu) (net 9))
 (via (at 140.208 124.46) (size 2.5) (drill 1) (layers F.Cu B.Cu) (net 7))
 (segment (start 140.796 124.46) (end 140.208 124.46) (width 0.5) (layer B.Cu) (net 7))
 (segment (start 143.002 120.904) (end 143.002 122.254) (width 0.5) (layer B.Cu) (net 7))
 (segment (start 143.002 122.254) (end 140.796 124.46) (width 0.5) (layer B.Cu) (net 7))
 (via (at 172.974 122.936) (size 2.5) (drill 1) (layers F.Cu B.Cu) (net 7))
 (segment (start 170.700001 125.209999) (end 172.974 122.936) (width 0.5) (layer F.Cu) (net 7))
 (segment (start 140.208 124.46) (end 140.957999 125.209999) (width 0.5) (layer F.Cu) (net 7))
 (segment (start 140.957999 125.209999) (end 170.700001 125.209999) (width 0.5) (layer F.Cu) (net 7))
 (segment (start 173.736 122.174) (end 178.816 122.174) (width 0.5) (layer B.Cu) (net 7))
 (segment (start 172.974 122.936) (end 173.736 122.174) (width 0.5) (layer B.Cu) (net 7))
 (segment (start 150.622 118.364) (end 151.824081 118.364) (width 0.5) (layer B.Cu) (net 4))
 (segment (start 150.622 118.364) (end 173.482 118.364) (width 0.5) (layer B.Cu) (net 4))
 (segment (start 174.752 119.634) (end 178.816 119.634) (width 0.5) (layer B.Cu) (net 4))
 (segment (start 173.482 118.364) (end 174.752 119.634) (width 0.5) (layer B.Cu) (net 4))
 (segment (start 124.968 127.762) (end 123.698 129.032) (width 0.5) (layer B.Cu) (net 10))
 (segment (start 124.968 122.174) (end 124.968 127.762) (width 0.5) (layer B.Cu) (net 10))
 (segment (start 129.794 129.032) (end 131.826 127) (width 0.5) (layer B.Cu) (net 10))
 (segment (start 123.698 129.032) (end 129.794 129.032) (width 0.5) (layer B.Cu) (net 10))
 (segment (start 148.082 120.904) (end 148.082 126.746) (width 0.5) (layer B.Cu) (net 5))
 (segment (start 151.566 123.262) (end 159.616 123.262) (width 0.5) (layer B.Cu) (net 5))
 (segment (start 148.082 126.746) (end 151.566 123.262) (width 0.5) (layer B.Cu) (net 5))
 (segment (start 148.082 116.078) (end 148.082 118.364) (width 0.5) (layer B.Cu) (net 1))
 (segment (start 145.288 113.284) (end 148.082 116.078) (width 0.5) (layer B.Cu) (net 1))
 (segment (start 132.08 115.824) (end 134.62 113.284) (width 0.5) (layer B.Cu) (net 1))
 (segment (start 134.62 113.284) (end 145.288 113.284) (width 0.5) (layer B.Cu) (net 1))
 (segment (start 149.352 114.808) (end 159.616 114.808) (width 0.5) (layer B.Cu) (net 1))
 (segment (start 148.082 116.078) (end 149.352 114.808) (width 0.5) (layer B.Cu) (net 1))
 (segment (start 161.030213 114.808) (end 166.116 114.808) (width 0.5) (layer B.Cu) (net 1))
 (segment (start 159.616 114.808) (end 161.030213 114.808) (width 0.5) (layer B.Cu) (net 1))
 (segment (start 145.542 116.84) (end 145.542 118.364) (width 0.5) (layer B.Cu) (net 3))
 (segment (start 135.636 115.824) (end 144.526 115.824) (width 0.5) (layer B.Cu) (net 3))
 (segment (start 144.526 115.824) (end 145.542 116.84) (width 0.5) (layer B.Cu) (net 3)))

